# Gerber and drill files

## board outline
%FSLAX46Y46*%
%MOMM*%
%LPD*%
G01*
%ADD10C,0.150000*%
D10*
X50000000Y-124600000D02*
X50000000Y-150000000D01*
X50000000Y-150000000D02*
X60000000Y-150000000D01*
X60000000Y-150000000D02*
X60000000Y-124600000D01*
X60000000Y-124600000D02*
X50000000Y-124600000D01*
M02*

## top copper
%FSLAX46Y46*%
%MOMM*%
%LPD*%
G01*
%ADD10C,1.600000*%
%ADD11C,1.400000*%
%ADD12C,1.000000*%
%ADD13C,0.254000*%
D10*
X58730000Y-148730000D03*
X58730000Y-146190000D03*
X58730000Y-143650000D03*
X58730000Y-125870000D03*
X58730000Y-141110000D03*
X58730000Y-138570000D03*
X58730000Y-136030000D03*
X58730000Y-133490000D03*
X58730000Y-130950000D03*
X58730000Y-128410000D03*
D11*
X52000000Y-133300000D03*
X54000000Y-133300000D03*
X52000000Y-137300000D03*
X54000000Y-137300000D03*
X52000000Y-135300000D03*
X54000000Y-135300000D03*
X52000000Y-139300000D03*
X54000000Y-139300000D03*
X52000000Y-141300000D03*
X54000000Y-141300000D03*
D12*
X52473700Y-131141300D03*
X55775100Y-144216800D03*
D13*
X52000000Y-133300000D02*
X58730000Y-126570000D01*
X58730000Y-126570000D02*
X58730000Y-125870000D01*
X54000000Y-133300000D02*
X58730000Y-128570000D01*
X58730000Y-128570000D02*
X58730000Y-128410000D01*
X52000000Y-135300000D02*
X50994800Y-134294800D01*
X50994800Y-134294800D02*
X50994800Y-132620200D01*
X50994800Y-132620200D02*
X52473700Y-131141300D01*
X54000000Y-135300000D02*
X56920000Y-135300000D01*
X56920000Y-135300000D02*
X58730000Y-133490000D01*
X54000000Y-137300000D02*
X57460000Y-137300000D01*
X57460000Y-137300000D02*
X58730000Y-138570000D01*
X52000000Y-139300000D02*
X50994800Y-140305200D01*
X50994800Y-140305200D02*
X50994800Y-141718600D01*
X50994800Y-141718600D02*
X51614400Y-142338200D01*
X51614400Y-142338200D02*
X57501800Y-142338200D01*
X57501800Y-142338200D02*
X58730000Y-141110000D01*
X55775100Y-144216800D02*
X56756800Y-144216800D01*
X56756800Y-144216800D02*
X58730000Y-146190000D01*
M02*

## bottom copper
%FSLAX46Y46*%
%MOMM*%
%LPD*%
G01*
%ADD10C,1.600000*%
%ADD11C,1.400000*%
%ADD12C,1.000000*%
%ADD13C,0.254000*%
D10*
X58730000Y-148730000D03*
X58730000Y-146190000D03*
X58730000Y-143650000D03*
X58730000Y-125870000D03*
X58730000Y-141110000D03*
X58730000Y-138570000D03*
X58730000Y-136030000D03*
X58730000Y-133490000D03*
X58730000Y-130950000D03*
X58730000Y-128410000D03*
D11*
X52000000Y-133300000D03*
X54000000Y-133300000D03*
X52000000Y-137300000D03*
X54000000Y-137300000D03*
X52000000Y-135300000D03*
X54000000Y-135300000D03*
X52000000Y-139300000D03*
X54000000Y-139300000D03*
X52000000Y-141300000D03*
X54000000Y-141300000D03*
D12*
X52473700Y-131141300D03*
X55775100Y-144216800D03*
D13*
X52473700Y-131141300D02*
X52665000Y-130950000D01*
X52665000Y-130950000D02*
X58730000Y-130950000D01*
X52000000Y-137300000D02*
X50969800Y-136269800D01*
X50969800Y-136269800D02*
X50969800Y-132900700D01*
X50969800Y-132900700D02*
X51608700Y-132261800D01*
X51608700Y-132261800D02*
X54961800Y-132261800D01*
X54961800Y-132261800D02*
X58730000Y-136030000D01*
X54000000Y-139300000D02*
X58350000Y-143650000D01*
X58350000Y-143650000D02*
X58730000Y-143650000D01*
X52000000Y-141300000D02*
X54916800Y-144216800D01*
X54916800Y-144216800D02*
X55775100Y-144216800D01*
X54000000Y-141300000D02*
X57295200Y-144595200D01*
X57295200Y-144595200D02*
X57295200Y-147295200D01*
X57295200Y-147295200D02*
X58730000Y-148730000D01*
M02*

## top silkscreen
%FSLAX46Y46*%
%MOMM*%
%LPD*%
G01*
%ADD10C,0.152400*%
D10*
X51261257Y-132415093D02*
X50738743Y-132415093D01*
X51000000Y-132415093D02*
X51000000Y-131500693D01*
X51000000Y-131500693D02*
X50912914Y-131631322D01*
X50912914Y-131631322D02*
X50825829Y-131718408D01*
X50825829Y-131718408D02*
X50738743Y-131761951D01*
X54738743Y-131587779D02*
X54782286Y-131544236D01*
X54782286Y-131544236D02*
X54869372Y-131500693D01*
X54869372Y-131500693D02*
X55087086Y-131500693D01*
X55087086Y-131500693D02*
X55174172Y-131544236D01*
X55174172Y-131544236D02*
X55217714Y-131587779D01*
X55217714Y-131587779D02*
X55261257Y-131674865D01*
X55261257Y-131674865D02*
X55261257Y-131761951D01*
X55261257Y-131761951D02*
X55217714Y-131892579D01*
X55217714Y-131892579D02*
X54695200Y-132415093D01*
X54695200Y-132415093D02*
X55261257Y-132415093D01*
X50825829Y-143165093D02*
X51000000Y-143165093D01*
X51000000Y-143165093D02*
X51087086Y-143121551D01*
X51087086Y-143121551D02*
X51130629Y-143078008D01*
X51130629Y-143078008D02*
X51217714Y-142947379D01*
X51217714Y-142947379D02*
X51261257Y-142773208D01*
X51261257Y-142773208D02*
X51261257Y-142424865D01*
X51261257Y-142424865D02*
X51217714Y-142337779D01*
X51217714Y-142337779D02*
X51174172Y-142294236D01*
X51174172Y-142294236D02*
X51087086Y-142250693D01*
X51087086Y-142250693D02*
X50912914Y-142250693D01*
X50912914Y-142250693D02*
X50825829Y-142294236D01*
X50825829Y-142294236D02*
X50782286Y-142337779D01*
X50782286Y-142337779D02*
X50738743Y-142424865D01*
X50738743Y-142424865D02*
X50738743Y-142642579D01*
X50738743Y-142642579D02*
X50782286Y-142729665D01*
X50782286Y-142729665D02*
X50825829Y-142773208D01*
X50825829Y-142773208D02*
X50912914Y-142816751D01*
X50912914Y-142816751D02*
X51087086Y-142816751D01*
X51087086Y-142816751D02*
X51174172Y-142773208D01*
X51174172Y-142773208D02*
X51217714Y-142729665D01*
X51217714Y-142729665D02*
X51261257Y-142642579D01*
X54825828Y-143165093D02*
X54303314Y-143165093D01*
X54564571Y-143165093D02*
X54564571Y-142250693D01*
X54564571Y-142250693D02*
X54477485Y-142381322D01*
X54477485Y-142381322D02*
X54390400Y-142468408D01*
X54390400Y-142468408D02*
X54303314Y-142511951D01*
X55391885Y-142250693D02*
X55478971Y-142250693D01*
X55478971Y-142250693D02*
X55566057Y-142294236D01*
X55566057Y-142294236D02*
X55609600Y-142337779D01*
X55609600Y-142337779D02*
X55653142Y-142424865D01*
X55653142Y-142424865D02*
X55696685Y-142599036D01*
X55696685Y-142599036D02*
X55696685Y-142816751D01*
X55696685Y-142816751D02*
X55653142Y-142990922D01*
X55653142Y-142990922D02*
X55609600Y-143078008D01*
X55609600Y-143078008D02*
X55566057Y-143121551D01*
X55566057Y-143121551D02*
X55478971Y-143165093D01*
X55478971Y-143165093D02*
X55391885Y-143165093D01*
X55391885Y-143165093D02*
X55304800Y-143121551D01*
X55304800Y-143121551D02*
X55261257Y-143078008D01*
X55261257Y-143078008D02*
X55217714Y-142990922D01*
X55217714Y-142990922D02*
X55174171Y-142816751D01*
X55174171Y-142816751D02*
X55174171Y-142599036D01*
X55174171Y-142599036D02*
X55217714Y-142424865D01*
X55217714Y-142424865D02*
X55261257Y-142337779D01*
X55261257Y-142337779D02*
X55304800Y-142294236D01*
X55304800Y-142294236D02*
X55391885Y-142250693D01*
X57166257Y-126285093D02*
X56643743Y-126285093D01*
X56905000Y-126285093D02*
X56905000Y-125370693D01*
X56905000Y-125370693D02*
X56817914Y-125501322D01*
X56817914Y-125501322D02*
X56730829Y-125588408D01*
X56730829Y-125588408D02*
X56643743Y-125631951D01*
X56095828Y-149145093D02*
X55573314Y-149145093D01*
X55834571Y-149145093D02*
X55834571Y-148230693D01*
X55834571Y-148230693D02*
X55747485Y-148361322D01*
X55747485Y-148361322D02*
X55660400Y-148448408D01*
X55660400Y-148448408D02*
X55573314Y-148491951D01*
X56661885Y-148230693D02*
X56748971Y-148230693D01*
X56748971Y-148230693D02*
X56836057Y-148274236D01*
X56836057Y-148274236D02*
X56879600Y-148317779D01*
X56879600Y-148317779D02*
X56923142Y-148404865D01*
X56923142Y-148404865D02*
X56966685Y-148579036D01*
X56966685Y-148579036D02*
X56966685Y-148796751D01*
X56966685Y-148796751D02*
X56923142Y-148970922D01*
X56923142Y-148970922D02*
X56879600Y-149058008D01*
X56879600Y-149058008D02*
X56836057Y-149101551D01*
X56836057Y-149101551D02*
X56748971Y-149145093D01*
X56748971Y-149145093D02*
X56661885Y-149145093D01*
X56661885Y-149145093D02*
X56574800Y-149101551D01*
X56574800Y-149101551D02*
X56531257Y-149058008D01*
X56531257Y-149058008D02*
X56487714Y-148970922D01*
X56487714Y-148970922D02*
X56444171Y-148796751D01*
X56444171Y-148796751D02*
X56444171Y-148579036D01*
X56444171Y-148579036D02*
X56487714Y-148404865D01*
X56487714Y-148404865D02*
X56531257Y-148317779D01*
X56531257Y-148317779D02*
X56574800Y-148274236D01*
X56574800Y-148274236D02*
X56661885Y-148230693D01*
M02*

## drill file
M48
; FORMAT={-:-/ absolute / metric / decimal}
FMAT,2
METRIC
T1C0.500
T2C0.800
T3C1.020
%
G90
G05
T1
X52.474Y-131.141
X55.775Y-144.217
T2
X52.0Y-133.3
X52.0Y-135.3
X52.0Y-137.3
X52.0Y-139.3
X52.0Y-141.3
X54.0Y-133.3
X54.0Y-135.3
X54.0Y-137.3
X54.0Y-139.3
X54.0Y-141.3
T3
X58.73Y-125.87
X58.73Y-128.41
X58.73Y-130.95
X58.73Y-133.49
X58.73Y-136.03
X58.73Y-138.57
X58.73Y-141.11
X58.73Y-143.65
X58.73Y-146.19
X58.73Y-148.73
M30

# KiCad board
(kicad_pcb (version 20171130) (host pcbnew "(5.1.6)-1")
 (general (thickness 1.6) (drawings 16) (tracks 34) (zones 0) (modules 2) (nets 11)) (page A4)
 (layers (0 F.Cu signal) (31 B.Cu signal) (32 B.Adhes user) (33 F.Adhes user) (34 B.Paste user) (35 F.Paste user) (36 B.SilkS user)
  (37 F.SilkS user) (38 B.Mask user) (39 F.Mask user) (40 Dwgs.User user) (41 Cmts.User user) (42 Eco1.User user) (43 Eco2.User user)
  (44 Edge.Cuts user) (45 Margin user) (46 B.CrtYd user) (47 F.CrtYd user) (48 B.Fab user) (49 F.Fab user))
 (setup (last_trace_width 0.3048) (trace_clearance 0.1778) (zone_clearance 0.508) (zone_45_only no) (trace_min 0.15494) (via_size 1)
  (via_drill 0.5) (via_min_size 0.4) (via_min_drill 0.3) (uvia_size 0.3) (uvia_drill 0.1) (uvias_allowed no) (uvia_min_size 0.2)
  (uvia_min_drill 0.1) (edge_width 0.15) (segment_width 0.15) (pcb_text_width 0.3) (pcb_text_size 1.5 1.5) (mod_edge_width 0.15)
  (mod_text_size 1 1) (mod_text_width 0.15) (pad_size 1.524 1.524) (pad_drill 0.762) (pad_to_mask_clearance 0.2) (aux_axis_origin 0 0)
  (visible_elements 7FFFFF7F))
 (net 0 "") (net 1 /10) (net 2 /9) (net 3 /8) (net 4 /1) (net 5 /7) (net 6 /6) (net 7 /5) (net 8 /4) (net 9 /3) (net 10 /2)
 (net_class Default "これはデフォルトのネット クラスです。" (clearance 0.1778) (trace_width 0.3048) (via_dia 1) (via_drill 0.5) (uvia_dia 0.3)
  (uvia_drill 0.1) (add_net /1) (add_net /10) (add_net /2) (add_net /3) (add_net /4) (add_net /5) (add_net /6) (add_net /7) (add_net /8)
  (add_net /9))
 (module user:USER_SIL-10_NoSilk (layer F.Cu) (at 58.73 137.3 270)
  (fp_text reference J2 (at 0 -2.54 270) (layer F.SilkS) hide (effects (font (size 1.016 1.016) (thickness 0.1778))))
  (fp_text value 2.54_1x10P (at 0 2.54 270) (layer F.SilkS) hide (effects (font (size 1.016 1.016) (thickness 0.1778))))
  (pad 10 thru_hole circle (at 11.43 0 270) (size 1.6 1.6) (drill 1.02) (layers *.Cu *.Mask) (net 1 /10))
  (pad 9 thru_hole circle (at 8.89 0 270) (size 1.6 1.6) (drill 1.02) (layers *.Cu *.Mask) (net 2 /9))
  (pad 8 thru_hole circle (at 6.35 0 270) (size 1.6 1.6) (drill 1.02) (layers *.Cu *.Mask) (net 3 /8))
  (pad 1 thru_hole circle (at -11.43 0 270) (size 1.6 1.6) (drill 1.02) (layers *.Cu *.Mask) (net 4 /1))
  (pad 7 thru_hole circle (at 3.81 0 270) (size 1.6 1.6) (drill 1.02) (layers *.Cu *.Mask) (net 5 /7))
  (pad 6 thru_hole circle (at 1.27 0 270) (size 1.6 1.6) (drill 1.02) (layers *.Cu *.Mask) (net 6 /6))
  (pad 5 thru_hole circle (at -1.27 0 270) (size 1.6 1.6) (drill 1.02) (layers *.Cu *.Mask) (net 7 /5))
  (pad 4 thru_hole circle (at -3.81 0 270) (size 1.6 1.6) (drill 1.02) (layers *.Cu *.Mask) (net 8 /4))
  (pad 3 thru_hole circle (at -6.35 0 270) (size 1.6 1.6) (drill 1.02) (layers *.Cu *.Mask) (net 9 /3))
  (pad 2 thru_hole circle (at -8.89 0 270) (size 1.6 1.6) (drill 1.02) (layers *.Cu *.Mask) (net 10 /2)))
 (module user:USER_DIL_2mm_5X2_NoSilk (layer F.Cu) (at 53 137.3)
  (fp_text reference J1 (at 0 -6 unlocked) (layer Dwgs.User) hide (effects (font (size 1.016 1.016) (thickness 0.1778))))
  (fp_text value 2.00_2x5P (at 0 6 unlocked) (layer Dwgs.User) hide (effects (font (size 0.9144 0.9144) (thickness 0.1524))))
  (pad 1 thru_hole circle (at -1 -4) (size 1.4 1.4) (drill 0.8) (layers *.Cu *.Mask) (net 4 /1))
  (pad 2 thru_hole circle (at 1 -4) (size 1.4 1.4) (drill 0.8) (layers *.Cu *.Mask) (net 10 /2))
  (pad 5 thru_hole circle (at -1 0) (size 1.4 1.4) (drill 0.8) (layers *.Cu *.Mask) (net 7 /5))
  (pad 6 thru_hole circle (at 1 0) (size 1.4 1.4) (drill 0.8) (layers *.Cu *.Mask) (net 6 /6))
  (pad 3 thru_hole circle (at -1 -2) (size 1.4 1.4) (drill 0.8) (layers *.Cu *.Mask) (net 9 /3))
  (pad 4 thru_hole circle (at 1 -2) (size 1.4 1.4) (drill 0.8) (layers *.Cu *.Mask) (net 8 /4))
  (pad 7 thru_hole circle (at -1 2) (size 1.4 1.4) (drill 0.8) (layers *.Cu *.Mask) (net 5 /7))
  (pad 8 thru_hole circle (at 1 2) (size 1.4 1.4) (drill 0.8) (layers *.Cu *.Mask) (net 3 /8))
  (pad 9 thru_hole circle (at -1 4) (size 1.4 1.4) (drill 0.8) (layers *.Cu *.Mask) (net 2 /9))
  (pad 10 thru_hole circle (at 1 4) (size 1.4 1.4) (drill 0.8) (layers *.Cu *.Mask) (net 1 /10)))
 (gr_line (start 50 124.6) (end 50 150) (angle 90) (layer Edge.Cuts) (width 0.15))
 (gr_line (start 50 150) (end 60 150) (angle 90) (layer Edge.Cuts) (width 0.15))
 (gr_line (start 60 150) (end 60 124.6) (angle 90) (layer Edge.Cuts) (width 0.15))
 (gr_line (start 60 124.6) (end 50 124.6) (angle 90) (layer Edge.Cuts) (width 0.15))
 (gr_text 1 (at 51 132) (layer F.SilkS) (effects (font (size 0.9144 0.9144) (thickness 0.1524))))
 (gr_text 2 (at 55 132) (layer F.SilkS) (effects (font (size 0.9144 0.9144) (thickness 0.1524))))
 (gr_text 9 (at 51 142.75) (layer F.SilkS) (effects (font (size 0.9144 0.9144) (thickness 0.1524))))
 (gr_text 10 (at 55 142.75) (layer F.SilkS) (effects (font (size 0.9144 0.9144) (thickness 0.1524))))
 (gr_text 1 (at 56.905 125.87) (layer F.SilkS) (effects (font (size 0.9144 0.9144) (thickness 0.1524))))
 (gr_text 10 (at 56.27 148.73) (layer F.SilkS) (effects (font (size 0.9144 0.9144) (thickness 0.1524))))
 (segment (start 52 133.3) (end 58.73 126.57) (width 0.254) (layer F.Cu) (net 4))
 (segment (start 58.73 126.57) (end 58.73 125.87) (width 0.254) (layer F.Cu) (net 4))
 (segment (start 54 133.3) (end 58.73 128.57) (width 0.254) (layer F.Cu) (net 10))
 (segment (start 58.73 128.57) (end 58.73 128.41) (width 0.254) (layer F.Cu) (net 10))
 (segment (start 52.4737 131.1413) (end 52.665 130.95) (width 0.254) (layer B.Cu) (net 9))
 (segment (start 52.665 130.95) (end 58.73 130.95) (width 0.254) (layer B.Cu) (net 9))
 (segment (start 52 135.3) (end 50.9948 134.2948) (width 0.254) (layer F.Cu) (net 9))
 (segment (start 50.9948 134.2948) (end 50.9948 132.6202) (width 0.254) (layer F.Cu) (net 9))
 (segment (start 50.9948 132.6202) (end 52.4737 131.1413) (width 0.254) (layer F.Cu) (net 9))
 (via (at 52.4737 131.1413) (size 1) (layers F.Cu B.Cu) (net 9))
 (segment (start 54 135.3) (end 56.92 135.3) (width 0.254) (layer F.Cu) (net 8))
 (segment (start 56.92 135.3) (end 58.73 133.49) (width 0.254) (layer F.Cu) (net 8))
 (segment (start 52 137.3) (end 50.9698 136.2698) (width 0.254) (layer B.Cu) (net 7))
 (segment (start 50.9698 136.2698) (end 50.9698 132.9007) (width 0.254) (layer B.Cu) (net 7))
 (segment (start 50.9698 132.9007) (end 51.6087 132.2618) (width 0.254) (layer B.Cu) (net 7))
 (segment (start 51.6087 132.2618) (end 54.9618 132.2618) (width 0.254) (layer B.Cu) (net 7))
 (segment (start 54.9618 132.2618) (end 58.73 136.03) (width 0.254) (layer B.Cu) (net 7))
 (segment (start 54 137.3) (end 57.46 137.3) (width 0.254) (layer F.Cu) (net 6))
 (segment (start 57.46 137.3) (end 58.73 138.57) (width 0.254) (layer F.Cu) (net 6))
 (segment (start 52 139.3) (end 50.9948 140.3052) (width 0.254) (layer F.Cu) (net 5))
 (segment (start 50.9948 140.3052) (end 50.9948 141.7186) (width 0.254) (layer F.Cu) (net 5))
 (segment (start 50.9948 141.7186) (end 51.6144 142.3382) (width 0.254) (layer F.Cu) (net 5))
 (segment (start 51.6144 142.3382) (end 57.5018 142.3382) (width 0.254) (layer F.Cu) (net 5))
 (segment (start 57.5018 142.3382) (end 58.73 141.11) (width 0.254) (layer F.Cu) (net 5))
 (segment (start 54 139.3) (end 58.35 143.65) (width 0.254) (layer B.Cu) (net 3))
 (segment (start 58.35 143.65) (end 58.73 143.65) (width 0.254) (layer B.Cu) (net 3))
 (segment (start 55.7751 144.2168) (end 56.7568 144.2168) (width 0.254) (layer F.Cu) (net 2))
 (segment (start 56.7568 144.2168) (end 58.73 146.19) (width 0.254) (layer F.Cu) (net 2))
 (segment (start 52 141.3) (end 54.9168 144.2168) (width 0.254) (layer B.Cu) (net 2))
 (segment (start 54.9168 144.2168) (end 55.7751 144.2168) (width 0.254) (layer B.Cu) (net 2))
 (via (at 55.7751 144.2168) (size 1) (layers F.Cu B.Cu) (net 2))
 (segment (start 54 141.3) (end 57.2952 144.5952) (width 0.254) (layer B.Cu) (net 1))
 (segment (start 57.2952 144.5952) (end 57.2952 147.2952) (width 0.254) (layer B.Cu) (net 1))
 (segment (start 57.2952 147.2952) (end 58.73 148.73) (width 0.254) (layer B.Cu) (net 1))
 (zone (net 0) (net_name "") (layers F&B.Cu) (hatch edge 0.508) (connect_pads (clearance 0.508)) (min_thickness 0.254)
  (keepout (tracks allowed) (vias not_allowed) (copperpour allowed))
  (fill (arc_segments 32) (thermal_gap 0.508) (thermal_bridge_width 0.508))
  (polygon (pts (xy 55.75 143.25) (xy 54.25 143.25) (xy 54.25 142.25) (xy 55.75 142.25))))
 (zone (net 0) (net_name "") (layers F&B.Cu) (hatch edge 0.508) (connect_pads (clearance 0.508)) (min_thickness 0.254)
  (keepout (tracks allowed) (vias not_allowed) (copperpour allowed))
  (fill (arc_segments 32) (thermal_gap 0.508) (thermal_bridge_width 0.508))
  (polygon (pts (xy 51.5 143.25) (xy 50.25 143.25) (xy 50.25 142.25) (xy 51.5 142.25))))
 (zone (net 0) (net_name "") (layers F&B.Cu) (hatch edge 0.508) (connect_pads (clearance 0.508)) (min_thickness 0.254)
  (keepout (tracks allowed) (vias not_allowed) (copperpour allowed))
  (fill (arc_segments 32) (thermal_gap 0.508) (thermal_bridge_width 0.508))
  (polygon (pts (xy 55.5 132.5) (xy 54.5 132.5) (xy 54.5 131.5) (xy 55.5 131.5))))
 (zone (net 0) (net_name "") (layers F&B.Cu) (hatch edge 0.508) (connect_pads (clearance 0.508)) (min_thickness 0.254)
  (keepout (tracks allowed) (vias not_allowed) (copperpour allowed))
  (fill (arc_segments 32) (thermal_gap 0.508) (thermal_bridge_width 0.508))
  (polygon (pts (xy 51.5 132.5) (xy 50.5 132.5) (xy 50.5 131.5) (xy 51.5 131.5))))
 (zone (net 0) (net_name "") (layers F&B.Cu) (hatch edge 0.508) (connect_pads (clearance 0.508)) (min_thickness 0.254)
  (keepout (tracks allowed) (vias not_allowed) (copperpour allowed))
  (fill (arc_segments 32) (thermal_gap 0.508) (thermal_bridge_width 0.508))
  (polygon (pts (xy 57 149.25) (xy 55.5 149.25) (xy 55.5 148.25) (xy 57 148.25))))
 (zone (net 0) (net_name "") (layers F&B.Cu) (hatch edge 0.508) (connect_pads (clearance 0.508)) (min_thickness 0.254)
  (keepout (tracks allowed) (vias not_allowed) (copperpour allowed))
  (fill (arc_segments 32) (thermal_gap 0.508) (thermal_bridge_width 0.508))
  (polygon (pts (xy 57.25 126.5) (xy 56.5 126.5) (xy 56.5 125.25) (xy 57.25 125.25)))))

